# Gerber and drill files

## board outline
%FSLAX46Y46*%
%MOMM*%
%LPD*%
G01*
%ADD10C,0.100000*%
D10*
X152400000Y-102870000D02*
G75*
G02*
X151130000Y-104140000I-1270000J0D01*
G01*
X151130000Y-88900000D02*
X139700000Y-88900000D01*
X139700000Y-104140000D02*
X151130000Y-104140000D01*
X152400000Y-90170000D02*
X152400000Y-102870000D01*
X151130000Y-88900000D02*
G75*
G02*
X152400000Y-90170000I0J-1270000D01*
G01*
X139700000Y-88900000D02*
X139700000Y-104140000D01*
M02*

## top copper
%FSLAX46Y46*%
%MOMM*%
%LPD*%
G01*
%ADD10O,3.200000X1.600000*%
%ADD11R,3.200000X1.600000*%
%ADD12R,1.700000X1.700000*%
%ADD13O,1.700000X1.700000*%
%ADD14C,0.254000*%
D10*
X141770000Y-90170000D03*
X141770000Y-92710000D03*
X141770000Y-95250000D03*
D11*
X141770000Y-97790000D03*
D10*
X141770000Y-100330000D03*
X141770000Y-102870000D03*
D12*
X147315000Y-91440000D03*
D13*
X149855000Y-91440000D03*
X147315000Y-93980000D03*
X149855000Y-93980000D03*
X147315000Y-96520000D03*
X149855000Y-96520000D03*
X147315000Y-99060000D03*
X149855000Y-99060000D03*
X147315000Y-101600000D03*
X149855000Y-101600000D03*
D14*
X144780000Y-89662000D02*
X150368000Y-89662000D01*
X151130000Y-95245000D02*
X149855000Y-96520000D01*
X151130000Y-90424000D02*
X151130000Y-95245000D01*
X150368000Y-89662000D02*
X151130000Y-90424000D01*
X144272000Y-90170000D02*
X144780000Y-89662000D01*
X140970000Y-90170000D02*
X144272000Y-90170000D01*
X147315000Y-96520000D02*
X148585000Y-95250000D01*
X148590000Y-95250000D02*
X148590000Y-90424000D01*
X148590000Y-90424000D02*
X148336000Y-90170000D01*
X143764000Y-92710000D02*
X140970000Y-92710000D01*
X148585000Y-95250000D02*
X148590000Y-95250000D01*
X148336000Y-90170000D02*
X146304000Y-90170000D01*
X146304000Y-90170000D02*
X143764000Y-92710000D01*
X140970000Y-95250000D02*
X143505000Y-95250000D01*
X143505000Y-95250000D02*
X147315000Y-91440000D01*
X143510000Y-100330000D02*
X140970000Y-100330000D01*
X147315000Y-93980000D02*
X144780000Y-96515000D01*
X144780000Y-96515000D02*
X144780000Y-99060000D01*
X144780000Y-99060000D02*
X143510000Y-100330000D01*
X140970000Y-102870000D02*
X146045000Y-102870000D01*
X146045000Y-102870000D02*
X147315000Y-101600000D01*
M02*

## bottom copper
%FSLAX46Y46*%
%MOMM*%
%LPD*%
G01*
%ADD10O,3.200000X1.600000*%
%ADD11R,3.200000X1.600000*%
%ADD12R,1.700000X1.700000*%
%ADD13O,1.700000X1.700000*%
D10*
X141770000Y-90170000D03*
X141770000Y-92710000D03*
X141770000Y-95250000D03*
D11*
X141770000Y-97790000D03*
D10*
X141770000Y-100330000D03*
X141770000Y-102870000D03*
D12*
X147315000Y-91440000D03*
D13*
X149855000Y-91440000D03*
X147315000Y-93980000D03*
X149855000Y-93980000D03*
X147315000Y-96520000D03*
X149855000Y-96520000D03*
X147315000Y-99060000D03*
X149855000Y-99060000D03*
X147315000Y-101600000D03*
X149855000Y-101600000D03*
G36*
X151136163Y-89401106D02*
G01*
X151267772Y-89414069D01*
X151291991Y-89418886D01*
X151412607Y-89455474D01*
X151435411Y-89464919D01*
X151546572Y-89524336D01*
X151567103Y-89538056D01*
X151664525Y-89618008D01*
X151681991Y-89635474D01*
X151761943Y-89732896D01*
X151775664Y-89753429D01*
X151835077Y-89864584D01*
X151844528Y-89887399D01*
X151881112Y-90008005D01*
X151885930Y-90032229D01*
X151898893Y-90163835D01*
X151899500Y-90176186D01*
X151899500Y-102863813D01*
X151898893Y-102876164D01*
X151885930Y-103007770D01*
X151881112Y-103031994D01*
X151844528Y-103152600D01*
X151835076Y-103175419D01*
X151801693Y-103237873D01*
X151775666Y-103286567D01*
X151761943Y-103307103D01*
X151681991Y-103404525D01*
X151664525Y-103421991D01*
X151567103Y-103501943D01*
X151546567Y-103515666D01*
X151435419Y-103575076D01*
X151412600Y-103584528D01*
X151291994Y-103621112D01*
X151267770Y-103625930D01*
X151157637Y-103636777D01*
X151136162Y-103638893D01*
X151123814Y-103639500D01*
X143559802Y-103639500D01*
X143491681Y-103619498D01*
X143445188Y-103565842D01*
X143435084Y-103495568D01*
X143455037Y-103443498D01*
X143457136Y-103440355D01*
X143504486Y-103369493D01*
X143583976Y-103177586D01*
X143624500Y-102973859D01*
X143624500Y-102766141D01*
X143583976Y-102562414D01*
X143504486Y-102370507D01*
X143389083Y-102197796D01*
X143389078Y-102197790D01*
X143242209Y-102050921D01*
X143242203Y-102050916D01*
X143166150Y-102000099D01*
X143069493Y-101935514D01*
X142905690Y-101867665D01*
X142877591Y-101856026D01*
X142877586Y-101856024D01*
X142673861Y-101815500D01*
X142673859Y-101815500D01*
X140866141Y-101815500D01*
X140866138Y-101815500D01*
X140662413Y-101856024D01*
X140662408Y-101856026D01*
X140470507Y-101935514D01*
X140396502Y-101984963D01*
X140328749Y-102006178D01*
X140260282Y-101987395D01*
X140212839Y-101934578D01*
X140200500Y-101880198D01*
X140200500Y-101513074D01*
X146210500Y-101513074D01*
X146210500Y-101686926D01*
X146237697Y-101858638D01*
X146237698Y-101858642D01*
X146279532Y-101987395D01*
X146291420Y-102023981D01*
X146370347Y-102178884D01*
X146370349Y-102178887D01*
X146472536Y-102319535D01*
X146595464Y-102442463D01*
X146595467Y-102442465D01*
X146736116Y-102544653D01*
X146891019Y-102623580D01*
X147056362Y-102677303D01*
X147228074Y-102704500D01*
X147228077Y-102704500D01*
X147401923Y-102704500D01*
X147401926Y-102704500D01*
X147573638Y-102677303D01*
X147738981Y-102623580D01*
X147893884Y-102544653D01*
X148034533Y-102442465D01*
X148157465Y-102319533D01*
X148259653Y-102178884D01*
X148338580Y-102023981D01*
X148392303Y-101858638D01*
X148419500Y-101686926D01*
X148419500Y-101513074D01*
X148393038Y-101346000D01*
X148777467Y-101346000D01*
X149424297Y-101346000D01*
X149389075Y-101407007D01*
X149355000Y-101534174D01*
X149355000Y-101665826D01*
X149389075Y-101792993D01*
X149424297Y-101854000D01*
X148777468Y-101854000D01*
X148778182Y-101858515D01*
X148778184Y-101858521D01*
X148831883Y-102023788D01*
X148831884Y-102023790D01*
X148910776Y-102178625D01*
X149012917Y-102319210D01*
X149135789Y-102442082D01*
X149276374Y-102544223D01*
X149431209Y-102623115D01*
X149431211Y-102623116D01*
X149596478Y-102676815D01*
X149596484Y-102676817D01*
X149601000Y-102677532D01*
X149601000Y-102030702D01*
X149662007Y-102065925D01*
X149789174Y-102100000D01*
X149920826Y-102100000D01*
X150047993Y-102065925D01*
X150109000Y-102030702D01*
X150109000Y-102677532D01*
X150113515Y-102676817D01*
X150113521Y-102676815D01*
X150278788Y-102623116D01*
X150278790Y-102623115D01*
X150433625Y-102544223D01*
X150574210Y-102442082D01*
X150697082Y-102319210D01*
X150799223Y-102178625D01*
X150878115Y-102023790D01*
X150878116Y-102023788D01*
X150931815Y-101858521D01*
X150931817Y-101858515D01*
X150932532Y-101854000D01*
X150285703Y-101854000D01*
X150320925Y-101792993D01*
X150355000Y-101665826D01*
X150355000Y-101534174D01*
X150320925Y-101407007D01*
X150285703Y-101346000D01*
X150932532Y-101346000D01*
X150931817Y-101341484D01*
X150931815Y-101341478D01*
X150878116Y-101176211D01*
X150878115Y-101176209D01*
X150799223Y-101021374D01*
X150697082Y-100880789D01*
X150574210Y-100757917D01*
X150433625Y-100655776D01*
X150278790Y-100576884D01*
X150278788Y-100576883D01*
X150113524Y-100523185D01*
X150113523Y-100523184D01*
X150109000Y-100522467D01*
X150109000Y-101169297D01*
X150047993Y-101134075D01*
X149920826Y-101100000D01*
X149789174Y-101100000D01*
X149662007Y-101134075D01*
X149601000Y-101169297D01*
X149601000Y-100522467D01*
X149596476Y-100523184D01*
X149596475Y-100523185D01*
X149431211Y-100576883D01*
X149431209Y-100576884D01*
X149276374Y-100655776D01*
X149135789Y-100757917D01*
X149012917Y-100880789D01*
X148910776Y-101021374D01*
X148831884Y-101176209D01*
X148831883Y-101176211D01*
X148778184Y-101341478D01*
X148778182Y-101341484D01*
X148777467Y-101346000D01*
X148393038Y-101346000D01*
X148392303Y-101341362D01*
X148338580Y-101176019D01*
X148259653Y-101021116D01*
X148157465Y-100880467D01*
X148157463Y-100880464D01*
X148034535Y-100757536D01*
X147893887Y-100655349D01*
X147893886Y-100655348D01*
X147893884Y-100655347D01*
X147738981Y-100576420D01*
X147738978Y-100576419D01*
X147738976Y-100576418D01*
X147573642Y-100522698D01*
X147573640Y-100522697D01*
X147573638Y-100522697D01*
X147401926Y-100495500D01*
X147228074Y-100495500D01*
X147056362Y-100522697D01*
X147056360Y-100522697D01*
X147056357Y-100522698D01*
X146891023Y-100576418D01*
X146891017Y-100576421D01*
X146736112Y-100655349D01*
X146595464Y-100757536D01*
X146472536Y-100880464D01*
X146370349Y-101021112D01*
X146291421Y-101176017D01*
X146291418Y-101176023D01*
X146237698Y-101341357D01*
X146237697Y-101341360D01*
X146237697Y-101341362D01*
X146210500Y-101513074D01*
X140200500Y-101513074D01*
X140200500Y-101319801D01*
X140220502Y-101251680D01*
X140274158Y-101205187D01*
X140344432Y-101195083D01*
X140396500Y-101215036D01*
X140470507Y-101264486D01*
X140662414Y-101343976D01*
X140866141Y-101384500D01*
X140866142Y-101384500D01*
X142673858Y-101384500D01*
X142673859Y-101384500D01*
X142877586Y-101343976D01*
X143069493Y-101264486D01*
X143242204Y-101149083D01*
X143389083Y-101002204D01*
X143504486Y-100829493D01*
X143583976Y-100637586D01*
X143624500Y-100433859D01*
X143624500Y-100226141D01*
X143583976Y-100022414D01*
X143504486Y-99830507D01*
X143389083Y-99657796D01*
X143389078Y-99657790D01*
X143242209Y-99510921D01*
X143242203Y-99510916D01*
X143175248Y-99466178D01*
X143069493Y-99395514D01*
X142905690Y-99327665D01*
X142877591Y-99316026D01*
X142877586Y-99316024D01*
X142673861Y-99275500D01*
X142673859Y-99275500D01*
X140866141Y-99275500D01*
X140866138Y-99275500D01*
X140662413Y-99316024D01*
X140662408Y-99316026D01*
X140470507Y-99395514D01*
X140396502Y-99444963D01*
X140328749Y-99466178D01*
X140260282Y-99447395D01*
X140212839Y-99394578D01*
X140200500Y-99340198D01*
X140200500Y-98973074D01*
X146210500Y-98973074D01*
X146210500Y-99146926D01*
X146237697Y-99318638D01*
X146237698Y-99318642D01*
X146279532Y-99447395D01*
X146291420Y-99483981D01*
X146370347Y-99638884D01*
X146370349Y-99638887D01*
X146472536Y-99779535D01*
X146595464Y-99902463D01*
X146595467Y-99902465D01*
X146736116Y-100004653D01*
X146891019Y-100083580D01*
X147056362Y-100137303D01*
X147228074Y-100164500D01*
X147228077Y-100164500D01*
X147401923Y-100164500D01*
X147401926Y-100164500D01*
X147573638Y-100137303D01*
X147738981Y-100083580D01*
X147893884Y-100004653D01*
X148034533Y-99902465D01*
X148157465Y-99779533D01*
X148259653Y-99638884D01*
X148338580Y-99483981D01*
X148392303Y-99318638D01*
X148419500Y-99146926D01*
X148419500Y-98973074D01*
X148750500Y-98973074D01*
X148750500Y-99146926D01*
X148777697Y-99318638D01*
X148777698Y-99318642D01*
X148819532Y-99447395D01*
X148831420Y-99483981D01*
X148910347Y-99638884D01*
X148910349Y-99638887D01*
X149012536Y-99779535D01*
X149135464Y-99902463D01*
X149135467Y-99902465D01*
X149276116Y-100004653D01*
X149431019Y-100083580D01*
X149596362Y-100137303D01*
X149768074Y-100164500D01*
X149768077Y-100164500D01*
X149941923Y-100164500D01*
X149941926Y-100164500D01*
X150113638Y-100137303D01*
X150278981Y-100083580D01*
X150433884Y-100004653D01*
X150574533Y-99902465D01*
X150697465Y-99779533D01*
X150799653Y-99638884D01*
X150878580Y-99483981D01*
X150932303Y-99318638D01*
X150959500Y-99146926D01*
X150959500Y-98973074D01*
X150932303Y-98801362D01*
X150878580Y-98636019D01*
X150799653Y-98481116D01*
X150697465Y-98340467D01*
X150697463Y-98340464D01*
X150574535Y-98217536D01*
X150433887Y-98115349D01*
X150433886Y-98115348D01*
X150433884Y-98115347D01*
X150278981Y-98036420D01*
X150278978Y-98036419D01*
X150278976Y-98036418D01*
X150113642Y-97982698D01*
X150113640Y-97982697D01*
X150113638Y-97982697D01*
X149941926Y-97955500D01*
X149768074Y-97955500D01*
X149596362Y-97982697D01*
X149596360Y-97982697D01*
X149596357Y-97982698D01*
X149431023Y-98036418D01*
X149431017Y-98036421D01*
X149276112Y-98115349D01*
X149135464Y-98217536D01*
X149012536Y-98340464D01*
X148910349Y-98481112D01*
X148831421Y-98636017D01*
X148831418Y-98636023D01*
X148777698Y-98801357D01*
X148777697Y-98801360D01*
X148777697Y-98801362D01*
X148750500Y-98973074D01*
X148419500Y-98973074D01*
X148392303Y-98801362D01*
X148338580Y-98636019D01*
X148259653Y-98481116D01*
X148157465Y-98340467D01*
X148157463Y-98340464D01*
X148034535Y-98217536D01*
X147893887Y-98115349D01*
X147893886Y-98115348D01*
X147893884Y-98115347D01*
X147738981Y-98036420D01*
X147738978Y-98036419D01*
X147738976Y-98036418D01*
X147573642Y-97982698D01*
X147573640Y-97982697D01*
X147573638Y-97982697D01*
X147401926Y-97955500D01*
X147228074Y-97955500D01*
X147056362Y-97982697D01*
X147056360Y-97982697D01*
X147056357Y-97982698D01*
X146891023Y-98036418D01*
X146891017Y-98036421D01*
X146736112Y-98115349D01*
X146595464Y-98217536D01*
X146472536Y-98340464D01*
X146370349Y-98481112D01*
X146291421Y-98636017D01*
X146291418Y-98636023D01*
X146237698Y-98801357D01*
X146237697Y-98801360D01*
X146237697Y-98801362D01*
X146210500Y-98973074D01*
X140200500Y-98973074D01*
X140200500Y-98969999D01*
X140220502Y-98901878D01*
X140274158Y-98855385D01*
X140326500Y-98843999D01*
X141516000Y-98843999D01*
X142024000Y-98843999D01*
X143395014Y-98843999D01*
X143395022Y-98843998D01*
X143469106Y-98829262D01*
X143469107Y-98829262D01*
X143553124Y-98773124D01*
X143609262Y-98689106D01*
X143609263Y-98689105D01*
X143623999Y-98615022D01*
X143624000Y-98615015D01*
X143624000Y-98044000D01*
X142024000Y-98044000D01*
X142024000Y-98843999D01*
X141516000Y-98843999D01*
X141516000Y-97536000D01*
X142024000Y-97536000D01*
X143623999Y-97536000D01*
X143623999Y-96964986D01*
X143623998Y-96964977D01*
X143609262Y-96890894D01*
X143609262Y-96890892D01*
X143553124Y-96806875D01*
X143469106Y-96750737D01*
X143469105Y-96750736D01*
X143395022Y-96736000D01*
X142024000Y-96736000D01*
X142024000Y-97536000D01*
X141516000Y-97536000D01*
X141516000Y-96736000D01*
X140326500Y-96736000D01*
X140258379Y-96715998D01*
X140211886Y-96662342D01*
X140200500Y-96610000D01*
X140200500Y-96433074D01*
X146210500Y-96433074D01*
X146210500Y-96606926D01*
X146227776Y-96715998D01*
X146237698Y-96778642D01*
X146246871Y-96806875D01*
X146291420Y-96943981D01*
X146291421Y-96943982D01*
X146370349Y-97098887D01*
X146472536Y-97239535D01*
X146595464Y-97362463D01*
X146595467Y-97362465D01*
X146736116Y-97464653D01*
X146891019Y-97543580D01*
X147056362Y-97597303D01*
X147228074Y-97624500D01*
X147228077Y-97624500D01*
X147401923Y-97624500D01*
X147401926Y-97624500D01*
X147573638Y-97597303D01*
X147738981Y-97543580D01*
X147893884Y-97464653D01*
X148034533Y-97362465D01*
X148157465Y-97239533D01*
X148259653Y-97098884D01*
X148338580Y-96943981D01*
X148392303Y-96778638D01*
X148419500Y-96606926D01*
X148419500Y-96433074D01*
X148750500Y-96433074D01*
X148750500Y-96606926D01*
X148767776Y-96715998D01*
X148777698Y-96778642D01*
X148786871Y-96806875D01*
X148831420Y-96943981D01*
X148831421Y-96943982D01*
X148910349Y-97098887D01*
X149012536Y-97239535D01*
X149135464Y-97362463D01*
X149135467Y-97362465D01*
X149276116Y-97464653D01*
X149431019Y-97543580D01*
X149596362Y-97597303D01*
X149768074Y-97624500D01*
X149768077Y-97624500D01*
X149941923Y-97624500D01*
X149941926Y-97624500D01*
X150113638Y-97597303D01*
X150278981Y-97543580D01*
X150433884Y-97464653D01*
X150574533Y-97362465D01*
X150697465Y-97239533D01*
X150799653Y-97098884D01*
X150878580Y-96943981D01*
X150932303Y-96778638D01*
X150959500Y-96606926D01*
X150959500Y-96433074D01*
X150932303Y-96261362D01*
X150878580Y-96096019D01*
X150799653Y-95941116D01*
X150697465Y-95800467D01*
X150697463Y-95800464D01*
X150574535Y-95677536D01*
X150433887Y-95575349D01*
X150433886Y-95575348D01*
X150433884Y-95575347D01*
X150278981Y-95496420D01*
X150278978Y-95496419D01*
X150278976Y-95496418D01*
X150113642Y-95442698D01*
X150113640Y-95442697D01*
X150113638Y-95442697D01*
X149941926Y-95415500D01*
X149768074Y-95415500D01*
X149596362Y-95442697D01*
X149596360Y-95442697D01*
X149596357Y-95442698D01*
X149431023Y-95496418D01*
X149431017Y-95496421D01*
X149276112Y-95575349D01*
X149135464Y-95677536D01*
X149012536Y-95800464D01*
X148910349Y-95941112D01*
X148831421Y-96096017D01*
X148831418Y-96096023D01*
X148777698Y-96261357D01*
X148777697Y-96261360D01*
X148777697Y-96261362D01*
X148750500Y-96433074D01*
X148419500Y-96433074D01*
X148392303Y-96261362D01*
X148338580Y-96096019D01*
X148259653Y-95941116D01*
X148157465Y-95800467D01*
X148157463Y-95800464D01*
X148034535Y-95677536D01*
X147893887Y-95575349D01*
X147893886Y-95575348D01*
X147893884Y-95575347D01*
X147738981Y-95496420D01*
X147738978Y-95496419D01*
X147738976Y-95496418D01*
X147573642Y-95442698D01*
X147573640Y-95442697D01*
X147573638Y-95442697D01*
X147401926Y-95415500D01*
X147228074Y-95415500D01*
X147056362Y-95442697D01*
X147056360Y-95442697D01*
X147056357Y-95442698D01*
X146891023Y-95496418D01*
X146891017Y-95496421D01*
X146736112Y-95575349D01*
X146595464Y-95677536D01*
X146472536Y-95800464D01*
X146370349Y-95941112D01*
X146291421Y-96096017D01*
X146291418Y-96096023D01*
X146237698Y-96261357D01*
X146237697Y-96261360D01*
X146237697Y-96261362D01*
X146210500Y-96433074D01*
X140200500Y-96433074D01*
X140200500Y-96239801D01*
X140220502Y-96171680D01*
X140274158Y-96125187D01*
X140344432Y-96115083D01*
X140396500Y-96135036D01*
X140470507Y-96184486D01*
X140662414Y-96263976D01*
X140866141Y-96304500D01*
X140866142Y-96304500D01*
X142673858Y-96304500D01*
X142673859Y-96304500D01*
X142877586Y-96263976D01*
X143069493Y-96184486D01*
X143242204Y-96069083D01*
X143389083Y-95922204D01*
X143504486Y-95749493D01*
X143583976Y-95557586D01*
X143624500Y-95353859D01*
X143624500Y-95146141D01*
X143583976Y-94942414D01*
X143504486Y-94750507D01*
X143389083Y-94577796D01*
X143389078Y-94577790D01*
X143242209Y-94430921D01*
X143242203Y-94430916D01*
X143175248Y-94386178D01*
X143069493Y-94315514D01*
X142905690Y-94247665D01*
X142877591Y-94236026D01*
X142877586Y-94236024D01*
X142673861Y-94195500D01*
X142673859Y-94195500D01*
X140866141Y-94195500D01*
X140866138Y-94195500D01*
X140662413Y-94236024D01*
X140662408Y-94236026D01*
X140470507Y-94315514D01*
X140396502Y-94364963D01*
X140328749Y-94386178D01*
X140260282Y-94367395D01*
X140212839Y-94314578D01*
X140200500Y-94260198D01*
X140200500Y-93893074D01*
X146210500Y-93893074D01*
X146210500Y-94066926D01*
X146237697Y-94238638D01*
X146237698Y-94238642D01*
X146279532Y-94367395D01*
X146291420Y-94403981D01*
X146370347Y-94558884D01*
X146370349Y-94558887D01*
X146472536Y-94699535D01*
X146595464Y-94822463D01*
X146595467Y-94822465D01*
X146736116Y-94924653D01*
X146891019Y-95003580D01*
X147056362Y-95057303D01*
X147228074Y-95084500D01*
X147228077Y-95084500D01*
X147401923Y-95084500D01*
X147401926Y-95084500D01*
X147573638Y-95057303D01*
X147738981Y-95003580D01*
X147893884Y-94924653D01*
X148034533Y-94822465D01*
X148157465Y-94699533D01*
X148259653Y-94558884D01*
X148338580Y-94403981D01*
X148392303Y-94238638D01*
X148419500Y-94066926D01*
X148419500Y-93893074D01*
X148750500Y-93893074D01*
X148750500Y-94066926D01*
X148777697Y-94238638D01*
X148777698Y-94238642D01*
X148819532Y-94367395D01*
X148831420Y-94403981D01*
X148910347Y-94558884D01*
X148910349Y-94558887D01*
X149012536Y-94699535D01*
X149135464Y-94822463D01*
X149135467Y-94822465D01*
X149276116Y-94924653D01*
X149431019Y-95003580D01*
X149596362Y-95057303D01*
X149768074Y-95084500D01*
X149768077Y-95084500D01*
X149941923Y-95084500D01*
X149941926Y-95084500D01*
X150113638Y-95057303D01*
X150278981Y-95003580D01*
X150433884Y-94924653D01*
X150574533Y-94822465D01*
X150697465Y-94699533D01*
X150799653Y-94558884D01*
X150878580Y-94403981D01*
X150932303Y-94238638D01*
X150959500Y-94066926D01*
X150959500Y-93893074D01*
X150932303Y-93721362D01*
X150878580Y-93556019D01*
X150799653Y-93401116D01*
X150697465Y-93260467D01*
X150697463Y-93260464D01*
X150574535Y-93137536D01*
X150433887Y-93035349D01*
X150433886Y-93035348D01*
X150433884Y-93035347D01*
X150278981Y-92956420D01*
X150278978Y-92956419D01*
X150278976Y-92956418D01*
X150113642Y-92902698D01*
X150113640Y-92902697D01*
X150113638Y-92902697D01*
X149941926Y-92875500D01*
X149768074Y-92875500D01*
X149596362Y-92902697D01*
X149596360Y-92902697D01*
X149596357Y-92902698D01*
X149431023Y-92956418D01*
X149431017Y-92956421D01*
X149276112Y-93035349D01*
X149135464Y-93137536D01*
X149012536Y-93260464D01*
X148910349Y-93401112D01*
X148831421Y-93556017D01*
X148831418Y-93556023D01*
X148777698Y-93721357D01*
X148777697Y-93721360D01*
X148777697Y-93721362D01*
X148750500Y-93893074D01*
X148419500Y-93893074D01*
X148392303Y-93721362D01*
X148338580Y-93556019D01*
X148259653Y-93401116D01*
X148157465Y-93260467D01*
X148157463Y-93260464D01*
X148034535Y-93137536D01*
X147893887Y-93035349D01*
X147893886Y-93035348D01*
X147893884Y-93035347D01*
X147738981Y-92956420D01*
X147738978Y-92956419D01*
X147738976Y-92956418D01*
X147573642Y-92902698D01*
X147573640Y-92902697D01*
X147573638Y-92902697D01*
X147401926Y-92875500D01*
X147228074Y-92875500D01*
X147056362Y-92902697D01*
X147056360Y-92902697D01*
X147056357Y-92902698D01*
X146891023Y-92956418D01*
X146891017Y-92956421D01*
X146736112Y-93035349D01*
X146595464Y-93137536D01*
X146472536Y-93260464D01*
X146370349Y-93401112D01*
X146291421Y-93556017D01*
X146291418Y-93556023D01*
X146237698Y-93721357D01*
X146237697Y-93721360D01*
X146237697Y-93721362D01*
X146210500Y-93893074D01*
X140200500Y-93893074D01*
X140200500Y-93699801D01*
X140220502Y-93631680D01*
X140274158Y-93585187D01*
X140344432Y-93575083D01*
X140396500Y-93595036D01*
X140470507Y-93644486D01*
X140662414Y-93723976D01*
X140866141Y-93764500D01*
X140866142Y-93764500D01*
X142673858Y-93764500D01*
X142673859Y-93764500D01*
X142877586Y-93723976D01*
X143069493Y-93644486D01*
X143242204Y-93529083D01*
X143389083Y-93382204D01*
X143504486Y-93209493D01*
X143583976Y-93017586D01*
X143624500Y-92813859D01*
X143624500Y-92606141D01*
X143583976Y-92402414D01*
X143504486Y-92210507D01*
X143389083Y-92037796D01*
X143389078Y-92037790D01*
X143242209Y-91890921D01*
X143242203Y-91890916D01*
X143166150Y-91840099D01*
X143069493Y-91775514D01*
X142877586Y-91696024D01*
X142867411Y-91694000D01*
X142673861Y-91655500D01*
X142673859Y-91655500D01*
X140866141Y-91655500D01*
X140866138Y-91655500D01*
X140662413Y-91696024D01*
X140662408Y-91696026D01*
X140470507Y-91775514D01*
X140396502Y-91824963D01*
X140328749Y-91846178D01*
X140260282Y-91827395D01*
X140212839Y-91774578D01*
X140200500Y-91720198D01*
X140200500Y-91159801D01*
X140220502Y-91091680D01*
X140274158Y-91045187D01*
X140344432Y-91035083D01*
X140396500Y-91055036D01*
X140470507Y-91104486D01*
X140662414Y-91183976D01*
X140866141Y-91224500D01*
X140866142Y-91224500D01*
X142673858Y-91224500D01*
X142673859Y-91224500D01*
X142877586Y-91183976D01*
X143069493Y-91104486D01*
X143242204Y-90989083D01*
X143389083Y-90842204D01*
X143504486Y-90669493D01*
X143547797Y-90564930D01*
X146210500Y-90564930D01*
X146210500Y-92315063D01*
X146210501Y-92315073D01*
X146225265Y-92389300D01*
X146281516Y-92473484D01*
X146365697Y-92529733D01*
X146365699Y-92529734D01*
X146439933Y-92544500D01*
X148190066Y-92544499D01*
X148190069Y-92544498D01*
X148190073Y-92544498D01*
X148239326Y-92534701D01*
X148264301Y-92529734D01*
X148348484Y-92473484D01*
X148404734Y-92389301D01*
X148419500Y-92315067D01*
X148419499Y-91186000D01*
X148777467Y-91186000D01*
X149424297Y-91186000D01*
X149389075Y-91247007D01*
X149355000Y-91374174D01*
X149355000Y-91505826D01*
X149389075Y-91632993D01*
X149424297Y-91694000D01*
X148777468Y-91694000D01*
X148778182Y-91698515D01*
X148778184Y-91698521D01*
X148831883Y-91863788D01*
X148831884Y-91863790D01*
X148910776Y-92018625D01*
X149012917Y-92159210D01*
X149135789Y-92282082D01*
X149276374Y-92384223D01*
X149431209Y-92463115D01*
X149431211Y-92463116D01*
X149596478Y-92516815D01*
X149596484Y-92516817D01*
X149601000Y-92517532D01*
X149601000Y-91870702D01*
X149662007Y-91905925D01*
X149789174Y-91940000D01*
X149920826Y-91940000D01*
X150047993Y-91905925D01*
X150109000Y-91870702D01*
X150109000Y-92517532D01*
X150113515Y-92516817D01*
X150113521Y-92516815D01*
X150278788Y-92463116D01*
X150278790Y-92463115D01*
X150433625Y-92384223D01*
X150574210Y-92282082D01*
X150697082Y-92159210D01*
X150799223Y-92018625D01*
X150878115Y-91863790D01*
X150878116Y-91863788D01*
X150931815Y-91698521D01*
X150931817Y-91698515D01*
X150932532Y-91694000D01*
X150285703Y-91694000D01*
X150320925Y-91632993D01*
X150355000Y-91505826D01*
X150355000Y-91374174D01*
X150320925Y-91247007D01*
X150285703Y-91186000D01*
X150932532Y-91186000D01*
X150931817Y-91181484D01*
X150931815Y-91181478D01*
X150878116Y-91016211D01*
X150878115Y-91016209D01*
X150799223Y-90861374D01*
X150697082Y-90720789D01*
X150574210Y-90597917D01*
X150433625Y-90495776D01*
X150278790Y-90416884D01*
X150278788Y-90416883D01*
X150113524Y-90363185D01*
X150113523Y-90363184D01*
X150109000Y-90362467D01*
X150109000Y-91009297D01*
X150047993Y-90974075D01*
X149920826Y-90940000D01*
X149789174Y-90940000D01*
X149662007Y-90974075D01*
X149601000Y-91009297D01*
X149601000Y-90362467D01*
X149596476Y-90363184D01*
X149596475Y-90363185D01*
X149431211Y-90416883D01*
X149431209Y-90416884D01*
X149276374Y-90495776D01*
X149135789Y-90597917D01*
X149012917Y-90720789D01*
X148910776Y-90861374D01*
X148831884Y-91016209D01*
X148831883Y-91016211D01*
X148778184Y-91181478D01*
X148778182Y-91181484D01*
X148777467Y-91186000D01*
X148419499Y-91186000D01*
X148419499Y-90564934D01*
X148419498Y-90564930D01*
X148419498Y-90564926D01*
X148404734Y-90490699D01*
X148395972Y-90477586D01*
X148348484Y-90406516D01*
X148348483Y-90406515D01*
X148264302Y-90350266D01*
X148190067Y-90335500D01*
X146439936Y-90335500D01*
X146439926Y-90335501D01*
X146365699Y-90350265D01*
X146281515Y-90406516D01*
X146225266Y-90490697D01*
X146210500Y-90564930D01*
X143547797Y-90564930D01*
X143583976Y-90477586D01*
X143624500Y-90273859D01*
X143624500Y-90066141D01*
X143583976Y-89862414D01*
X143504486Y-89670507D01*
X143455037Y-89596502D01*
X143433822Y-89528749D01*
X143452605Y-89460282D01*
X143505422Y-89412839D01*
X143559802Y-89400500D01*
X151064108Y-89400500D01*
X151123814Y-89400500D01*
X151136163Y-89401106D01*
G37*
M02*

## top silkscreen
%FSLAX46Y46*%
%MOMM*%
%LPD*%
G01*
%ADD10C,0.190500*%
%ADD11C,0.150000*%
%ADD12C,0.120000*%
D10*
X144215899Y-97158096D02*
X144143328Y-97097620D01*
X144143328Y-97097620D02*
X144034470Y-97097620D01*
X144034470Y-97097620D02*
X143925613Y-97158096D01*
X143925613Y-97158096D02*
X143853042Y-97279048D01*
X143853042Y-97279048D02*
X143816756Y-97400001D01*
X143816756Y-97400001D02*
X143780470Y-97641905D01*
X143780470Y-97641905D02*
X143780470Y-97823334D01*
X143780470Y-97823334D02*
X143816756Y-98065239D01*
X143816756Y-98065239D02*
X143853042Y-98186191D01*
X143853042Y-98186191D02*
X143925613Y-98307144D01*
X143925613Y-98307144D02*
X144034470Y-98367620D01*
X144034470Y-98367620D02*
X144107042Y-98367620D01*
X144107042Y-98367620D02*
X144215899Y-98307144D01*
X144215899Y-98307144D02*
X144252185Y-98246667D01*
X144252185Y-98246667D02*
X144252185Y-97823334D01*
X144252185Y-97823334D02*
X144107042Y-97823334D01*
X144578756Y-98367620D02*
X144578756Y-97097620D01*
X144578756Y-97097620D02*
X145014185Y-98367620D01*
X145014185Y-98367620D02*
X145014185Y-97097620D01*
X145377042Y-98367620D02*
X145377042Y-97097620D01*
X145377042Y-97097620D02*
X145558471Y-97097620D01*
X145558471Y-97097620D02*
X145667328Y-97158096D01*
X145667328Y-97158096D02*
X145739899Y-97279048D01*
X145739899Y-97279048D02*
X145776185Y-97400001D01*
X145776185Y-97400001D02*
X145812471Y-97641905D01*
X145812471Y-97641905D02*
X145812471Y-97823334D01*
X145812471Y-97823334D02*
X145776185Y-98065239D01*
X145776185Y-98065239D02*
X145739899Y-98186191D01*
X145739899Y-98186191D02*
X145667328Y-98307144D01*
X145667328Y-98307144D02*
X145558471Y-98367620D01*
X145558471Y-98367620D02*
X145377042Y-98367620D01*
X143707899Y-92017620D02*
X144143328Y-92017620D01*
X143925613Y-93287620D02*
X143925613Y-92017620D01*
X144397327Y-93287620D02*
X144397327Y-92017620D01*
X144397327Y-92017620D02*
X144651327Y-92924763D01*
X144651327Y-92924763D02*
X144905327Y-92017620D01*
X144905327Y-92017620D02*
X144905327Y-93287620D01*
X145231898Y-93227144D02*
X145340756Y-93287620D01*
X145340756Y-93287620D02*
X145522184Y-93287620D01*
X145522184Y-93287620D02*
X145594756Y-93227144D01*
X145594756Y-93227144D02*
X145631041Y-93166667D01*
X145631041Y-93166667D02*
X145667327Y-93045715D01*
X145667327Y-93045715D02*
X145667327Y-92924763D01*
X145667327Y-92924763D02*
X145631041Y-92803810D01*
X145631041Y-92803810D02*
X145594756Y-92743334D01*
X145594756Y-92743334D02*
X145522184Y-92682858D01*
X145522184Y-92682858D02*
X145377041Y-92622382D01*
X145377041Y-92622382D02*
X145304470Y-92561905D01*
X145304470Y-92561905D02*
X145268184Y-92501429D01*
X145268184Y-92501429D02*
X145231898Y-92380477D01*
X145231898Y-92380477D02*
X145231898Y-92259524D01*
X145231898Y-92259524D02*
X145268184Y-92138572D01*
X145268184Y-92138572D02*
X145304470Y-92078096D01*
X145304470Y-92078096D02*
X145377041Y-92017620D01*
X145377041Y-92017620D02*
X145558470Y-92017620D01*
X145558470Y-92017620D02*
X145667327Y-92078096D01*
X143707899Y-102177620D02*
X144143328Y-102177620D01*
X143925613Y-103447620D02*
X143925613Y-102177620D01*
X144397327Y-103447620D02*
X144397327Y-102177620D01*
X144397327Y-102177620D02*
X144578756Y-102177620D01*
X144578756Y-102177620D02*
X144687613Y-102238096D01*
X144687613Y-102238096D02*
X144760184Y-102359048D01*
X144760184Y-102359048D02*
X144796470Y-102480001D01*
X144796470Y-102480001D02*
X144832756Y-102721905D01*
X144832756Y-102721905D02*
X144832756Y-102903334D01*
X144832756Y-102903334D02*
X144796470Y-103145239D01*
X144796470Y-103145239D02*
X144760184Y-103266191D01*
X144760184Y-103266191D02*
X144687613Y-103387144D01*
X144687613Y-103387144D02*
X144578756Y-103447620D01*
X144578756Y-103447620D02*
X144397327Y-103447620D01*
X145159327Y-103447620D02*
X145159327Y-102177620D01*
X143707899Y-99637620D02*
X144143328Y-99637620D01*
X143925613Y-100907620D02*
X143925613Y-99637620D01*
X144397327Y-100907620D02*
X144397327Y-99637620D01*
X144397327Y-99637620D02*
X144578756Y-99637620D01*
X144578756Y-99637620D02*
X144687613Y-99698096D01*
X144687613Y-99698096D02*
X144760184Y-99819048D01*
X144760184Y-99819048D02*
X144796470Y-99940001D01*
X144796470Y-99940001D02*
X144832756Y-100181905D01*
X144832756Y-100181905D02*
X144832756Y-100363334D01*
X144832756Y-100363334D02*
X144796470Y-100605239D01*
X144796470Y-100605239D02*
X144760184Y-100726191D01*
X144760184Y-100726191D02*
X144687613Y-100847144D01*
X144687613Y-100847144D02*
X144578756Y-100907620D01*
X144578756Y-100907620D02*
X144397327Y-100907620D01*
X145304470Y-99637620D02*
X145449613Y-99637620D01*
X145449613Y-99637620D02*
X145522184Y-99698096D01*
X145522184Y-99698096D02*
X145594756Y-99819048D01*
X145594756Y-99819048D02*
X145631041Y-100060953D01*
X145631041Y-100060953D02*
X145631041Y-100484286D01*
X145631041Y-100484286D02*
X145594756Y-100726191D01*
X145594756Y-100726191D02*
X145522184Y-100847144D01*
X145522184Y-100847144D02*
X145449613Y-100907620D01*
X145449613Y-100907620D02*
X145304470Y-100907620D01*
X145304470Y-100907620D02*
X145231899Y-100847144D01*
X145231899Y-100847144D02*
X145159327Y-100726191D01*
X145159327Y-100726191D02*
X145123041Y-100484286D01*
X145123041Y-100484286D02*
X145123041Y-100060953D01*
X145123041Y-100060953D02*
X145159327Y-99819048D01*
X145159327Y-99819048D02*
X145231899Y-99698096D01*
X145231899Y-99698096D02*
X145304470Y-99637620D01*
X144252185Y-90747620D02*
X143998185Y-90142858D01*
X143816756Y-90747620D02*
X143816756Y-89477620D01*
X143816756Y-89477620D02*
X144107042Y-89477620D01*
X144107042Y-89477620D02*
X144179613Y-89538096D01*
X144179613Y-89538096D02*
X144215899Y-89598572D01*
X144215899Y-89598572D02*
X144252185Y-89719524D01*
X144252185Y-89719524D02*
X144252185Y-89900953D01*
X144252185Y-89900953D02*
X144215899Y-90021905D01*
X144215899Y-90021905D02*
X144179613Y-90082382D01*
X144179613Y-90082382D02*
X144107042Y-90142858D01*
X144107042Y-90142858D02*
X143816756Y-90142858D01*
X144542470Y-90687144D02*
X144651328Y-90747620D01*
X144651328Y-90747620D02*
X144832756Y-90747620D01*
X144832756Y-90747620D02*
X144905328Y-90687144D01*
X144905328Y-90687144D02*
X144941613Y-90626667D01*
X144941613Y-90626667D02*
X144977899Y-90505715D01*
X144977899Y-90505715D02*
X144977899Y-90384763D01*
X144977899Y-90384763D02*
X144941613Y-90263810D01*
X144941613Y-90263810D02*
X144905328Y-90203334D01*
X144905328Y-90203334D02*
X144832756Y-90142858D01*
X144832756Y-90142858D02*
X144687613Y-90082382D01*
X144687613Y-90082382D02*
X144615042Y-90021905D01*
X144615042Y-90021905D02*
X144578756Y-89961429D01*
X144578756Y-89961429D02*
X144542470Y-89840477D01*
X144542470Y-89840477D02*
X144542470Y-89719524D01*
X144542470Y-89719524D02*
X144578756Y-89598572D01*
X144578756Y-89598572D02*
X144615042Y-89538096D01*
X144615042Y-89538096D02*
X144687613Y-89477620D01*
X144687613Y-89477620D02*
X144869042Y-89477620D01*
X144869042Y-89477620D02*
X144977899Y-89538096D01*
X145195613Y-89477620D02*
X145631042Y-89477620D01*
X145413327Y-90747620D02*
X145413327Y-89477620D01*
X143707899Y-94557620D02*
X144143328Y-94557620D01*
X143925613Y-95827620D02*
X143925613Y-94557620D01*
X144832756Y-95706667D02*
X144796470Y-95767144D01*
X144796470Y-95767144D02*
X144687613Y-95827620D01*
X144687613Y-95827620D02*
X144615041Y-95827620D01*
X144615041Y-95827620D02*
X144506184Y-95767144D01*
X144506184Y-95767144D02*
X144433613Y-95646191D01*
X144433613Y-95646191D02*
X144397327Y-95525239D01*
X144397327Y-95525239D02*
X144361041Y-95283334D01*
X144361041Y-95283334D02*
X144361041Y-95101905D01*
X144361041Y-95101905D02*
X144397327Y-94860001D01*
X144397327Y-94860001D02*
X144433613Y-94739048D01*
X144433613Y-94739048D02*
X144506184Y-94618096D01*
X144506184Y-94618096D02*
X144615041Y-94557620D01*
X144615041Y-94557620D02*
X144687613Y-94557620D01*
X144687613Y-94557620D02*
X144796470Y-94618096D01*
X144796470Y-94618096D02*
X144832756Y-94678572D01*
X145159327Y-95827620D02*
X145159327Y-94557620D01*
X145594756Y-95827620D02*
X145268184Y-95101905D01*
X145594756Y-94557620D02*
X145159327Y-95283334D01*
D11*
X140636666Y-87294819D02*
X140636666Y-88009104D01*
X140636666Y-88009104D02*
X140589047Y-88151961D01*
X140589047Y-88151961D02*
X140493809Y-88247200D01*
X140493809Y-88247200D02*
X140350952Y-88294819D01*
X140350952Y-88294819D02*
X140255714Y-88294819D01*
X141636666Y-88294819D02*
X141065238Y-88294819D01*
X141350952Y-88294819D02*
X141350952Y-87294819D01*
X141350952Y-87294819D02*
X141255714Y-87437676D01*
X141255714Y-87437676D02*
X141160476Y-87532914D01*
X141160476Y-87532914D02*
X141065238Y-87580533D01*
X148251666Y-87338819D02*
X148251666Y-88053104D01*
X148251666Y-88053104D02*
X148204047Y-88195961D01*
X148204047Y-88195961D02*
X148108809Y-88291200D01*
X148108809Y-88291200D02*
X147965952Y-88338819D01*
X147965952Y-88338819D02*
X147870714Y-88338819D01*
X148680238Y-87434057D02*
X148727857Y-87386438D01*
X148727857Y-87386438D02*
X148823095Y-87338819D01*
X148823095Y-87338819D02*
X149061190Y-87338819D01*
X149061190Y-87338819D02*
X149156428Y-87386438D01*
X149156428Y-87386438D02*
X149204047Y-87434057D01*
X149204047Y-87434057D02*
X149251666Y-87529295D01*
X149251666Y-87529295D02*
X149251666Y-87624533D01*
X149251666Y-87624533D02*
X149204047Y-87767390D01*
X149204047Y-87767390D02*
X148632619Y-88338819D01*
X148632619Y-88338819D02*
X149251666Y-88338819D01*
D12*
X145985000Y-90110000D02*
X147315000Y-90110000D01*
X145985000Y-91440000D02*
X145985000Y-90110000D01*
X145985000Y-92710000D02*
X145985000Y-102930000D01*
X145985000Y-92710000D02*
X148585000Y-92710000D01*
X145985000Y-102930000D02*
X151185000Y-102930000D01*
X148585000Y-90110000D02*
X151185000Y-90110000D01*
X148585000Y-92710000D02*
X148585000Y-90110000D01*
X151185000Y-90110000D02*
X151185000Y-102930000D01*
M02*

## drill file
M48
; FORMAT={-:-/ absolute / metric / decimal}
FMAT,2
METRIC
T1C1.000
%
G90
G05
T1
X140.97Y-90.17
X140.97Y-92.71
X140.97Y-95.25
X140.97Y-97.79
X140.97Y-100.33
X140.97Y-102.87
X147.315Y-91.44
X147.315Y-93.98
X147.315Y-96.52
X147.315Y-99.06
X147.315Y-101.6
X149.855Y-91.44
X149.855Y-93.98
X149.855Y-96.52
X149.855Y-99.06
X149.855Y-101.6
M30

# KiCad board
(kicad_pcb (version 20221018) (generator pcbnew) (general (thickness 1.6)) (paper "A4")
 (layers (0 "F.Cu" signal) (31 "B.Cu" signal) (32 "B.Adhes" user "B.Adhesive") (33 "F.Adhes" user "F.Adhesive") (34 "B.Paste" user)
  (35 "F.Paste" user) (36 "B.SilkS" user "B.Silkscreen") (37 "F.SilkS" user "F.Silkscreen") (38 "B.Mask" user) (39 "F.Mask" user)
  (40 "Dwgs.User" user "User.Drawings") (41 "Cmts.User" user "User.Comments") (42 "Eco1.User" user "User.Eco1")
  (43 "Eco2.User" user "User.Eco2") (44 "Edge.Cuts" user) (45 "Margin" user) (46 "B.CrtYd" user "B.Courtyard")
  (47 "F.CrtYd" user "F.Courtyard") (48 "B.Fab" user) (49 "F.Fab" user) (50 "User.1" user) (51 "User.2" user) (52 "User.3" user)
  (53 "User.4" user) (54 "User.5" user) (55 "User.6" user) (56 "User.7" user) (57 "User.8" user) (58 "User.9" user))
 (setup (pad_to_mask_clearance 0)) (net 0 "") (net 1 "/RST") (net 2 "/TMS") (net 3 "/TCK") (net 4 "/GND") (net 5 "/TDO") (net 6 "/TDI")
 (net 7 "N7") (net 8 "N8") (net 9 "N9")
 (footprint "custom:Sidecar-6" (layer "F.Cu") (at 140.97 90.17)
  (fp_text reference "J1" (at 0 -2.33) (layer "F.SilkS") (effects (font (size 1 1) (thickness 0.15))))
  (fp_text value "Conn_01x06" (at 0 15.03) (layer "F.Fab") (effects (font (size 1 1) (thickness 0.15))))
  (pad "1" thru_hole oval (at 0 0) (size 3.2 1.6) (drill 1 (offset 0.8 0)) (layers "*.Cu" "*.Mask") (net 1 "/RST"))
  (pad "2" thru_hole oval (at 0 2.54) (size 3.2 1.6) (drill 1 (offset 0.8 0)) (layers "*.Cu" "*.Mask") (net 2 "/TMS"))
  (pad "3" thru_hole oval (at 0 5.08) (size 3.2 1.6) (drill 1 (offset 0.8 0)) (layers "*.Cu" "*.Mask") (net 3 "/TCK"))
  (pad "4" thru_hole rect (at 0 7.62) (size 3.2 1.6) (drill 1 (offset 0.8 0)) (layers "*.Cu" "*.Mask") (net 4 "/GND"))
  (pad "5" thru_hole oval (at 0 10.16) (size 3.2 1.6) (drill 1 (offset 0.8 0)) (layers "*.Cu" "*.Mask") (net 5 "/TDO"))
  (pad "6" thru_hole oval (at 0 12.7) (size 3.2 1.6) (drill 1 (offset 0.8 0)) (layers "*.Cu" "*.Mask") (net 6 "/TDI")))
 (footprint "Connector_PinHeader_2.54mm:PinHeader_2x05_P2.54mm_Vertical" (layer "F.Cu") (at 147.315 91.44)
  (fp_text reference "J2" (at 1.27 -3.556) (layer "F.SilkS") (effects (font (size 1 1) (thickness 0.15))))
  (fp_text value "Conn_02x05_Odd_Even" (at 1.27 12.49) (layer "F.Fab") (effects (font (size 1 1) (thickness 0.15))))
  (fp_line (start -1.33 -1.33) (end 0 -1.33) (stroke (width 0.12) (type solid)) (layer "F.SilkS"))
  (fp_line (start -1.33 0) (end -1.33 -1.33) (stroke (width 0.12) (type solid)) (layer "F.SilkS"))
  (fp_line (start -1.33 1.27) (end -1.33 11.49) (stroke (width 0.12) (type solid)) (layer "F.SilkS"))
  (fp_line (start -1.33 1.27) (end 1.27 1.27) (stroke (width 0.12) (type solid)) (layer "F.SilkS"))
  (fp_line (start -1.33 11.49) (end 3.87 11.49) (stroke (width 0.12) (type solid)) (layer "F.SilkS"))
  (fp_line (start 1.27 -1.33) (end 3.87 -1.33) (stroke (width 0.12) (type solid)) (layer "F.SilkS"))
  (fp_line (start 1.27 1.27) (end 1.27 -1.33) (stroke (width 0.12) (type solid)) (layer "F.SilkS"))
  (fp_line (start 3.87 -1.33) (end 3.87 11.49) (stroke (width 0.12) (type solid)) (layer "F.SilkS"))
  (pad "1" thru_hole rect (at 0 0) (size 1.7 1.7) (drill 1) (layers "*.Cu" "*.Mask") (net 3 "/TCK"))
  (pad "2" thru_hole oval (at 2.54 0) (size 1.7 1.7) (drill 1) (layers "*.Cu" "*.Mask") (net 4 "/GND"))
  (pad "3" thru_hole oval (at 0 2.54) (size 1.7 1.7) (drill 1) (layers "*.Cu" "*.Mask") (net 5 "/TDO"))
  (pad "4" thru_hole oval (at 2.54 2.54) (size 1.7 1.7) (drill 1) (layers "*.Cu" "*.Mask") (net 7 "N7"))
  (pad "5" thru_hole oval (at 0 5.08) (size 1.7 1.7) (drill 1) (layers "*.Cu" "*.Mask") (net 2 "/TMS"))
  (pad "6" thru_hole oval (at 2.54 5.08) (size 1.7 1.7) (drill 1) (layers "*.Cu" "*.Mask") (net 1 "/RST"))
  (pad "7" thru_hole oval (at 0 7.62) (size 1.7 1.7) (drill 1) (layers "*.Cu" "*.Mask") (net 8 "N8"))
  (pad "8" thru_hole oval (at 2.54 7.62) (size 1.7 1.7) (drill 1) (layers "*.Cu" "*.Mask") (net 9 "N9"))
  (pad "9" thru_hole oval (at 0 10.16) (size 1.7 1.7) (drill 1) (layers "*.Cu" "*.Mask") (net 6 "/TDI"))
  (pad "10" thru_hole oval (at 2.54 10.16) (size 1.7 1.7) (drill 1) (layers "*.Cu" "*.Mask") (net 4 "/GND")))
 (gr_arc (start 152.4 102.87) (mid 152.028026 103.768026) (end 151.13 104.14) (stroke (width 0.1) (type default)) (layer "Edge.Cuts"))
 (gr_line (start 151.13 88.9) (end 139.7 88.9) (stroke (width 0.1) (type default)) (layer "Edge.Cuts"))
 (gr_line (start 139.7 104.14) (end 151.13 104.14) (stroke (width 0.1) (type default)) (layer "Edge.Cuts"))
 (gr_line (start 152.4 90.17) (end 152.4 102.87) (stroke (width 0.1) (type default)) (layer "Edge.Cuts"))
 (gr_arc (start 151.13 88.9) (mid 152.028026 89.271974) (end 152.4 90.17) (stroke (width 0.1) (type default)) (layer "Edge.Cuts"))
 (gr_line (start 139.7 88.9) (end 139.7 104.14) (stroke (width 0.1) (type default)) (layer "Edge.Cuts"))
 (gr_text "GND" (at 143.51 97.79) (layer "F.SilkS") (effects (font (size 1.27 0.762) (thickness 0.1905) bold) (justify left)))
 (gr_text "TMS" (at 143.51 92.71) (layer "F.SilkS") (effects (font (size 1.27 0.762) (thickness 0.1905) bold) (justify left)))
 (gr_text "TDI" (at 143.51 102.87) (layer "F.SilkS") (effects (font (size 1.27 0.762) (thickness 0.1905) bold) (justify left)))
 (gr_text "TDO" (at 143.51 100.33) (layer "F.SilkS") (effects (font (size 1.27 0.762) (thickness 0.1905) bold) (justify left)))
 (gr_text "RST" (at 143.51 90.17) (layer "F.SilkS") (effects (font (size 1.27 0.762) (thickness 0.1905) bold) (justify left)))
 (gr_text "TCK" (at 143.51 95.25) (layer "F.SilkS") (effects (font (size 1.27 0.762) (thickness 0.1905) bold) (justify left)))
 (segment (start 144.78 89.662) (end 150.368 89.662) (width 0.254) (layer "F.Cu") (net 1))
 (segment (start 151.13 95.245) (end 149.855 96.52) (width 0.254) (layer "F.Cu") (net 1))
 (segment (start 151.13 90.424) (end 151.13 95.245) (width 0.254) (layer "F.Cu") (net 1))
 (segment (start 150.368 89.662) (end 151.13 90.424) (width 0.254) (layer "F.Cu") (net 1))
 (segment (start 144.272 90.17) (end 144.78 89.662) (width 0.254) (layer "F.Cu") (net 1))
 (segment (start 140.97 90.17) (end 144.272 90.17) (width 0.254) (layer "F.Cu") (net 1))
 (segment (start 147.315 96.52) (end 148.585 95.25) (width 0.254) (layer "F.Cu") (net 2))
 (segment (start 148.59 95.25) (end 148.59 90.424) (width 0.254) (layer "F.Cu") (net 2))
 (segment (start 148.59 90.424) (end 148.336 90.17) (width 0.254) (layer "F.Cu") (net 2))
 (segment (start 143.764 92.71) (end 140.97 92.71) (width 0.254) (layer "F.Cu") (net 2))
 (segment (start 148.585 95.25) (end 148.59 95.25) (width 0.254) (layer "F.Cu") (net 2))
 (segment (start 148.336 90.17) (end 146.304 90.17) (width 0.254) (layer "F.Cu") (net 2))
 (segment (start 146.304 90.17) (end 143.764 92.71) (width 0.254) (layer "F.Cu") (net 2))
 (segment (start 140.97 95.25) (end 143.505 95.25) (width 0.254) (layer "F.Cu") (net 3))
 (segment (start 143.505 95.25) (end 147.315 91.44) (width 0.254) (layer "F.Cu") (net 3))
 (segment (start 143.51 100.33) (end 140.97 100.33) (width 0.254) (layer "F.Cu") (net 5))
 (segment (start 147.315 93.98) (end 144.78 96.515) (width 0.254) (layer "F.Cu") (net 5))
 (segment (start 144.78 96.515) (end 144.78 99.06) (width 0.254) (layer "F.Cu") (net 5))
 (segment (start 144.78 99.06) (end 143.51 100.33) (width 0.254) (layer "F.Cu") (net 5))
 (segment (start 140.97 102.87) (end 146.045 102.87) (width 0.254) (layer "F.Cu") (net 6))
 (segment (start 146.045 102.87) (end 147.315 101.6) (width 0.254) (layer "F.Cu") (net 6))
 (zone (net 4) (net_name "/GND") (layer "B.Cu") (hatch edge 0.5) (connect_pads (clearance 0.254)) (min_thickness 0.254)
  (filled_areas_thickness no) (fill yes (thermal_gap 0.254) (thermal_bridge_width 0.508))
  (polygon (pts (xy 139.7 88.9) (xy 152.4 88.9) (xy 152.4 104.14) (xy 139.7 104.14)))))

